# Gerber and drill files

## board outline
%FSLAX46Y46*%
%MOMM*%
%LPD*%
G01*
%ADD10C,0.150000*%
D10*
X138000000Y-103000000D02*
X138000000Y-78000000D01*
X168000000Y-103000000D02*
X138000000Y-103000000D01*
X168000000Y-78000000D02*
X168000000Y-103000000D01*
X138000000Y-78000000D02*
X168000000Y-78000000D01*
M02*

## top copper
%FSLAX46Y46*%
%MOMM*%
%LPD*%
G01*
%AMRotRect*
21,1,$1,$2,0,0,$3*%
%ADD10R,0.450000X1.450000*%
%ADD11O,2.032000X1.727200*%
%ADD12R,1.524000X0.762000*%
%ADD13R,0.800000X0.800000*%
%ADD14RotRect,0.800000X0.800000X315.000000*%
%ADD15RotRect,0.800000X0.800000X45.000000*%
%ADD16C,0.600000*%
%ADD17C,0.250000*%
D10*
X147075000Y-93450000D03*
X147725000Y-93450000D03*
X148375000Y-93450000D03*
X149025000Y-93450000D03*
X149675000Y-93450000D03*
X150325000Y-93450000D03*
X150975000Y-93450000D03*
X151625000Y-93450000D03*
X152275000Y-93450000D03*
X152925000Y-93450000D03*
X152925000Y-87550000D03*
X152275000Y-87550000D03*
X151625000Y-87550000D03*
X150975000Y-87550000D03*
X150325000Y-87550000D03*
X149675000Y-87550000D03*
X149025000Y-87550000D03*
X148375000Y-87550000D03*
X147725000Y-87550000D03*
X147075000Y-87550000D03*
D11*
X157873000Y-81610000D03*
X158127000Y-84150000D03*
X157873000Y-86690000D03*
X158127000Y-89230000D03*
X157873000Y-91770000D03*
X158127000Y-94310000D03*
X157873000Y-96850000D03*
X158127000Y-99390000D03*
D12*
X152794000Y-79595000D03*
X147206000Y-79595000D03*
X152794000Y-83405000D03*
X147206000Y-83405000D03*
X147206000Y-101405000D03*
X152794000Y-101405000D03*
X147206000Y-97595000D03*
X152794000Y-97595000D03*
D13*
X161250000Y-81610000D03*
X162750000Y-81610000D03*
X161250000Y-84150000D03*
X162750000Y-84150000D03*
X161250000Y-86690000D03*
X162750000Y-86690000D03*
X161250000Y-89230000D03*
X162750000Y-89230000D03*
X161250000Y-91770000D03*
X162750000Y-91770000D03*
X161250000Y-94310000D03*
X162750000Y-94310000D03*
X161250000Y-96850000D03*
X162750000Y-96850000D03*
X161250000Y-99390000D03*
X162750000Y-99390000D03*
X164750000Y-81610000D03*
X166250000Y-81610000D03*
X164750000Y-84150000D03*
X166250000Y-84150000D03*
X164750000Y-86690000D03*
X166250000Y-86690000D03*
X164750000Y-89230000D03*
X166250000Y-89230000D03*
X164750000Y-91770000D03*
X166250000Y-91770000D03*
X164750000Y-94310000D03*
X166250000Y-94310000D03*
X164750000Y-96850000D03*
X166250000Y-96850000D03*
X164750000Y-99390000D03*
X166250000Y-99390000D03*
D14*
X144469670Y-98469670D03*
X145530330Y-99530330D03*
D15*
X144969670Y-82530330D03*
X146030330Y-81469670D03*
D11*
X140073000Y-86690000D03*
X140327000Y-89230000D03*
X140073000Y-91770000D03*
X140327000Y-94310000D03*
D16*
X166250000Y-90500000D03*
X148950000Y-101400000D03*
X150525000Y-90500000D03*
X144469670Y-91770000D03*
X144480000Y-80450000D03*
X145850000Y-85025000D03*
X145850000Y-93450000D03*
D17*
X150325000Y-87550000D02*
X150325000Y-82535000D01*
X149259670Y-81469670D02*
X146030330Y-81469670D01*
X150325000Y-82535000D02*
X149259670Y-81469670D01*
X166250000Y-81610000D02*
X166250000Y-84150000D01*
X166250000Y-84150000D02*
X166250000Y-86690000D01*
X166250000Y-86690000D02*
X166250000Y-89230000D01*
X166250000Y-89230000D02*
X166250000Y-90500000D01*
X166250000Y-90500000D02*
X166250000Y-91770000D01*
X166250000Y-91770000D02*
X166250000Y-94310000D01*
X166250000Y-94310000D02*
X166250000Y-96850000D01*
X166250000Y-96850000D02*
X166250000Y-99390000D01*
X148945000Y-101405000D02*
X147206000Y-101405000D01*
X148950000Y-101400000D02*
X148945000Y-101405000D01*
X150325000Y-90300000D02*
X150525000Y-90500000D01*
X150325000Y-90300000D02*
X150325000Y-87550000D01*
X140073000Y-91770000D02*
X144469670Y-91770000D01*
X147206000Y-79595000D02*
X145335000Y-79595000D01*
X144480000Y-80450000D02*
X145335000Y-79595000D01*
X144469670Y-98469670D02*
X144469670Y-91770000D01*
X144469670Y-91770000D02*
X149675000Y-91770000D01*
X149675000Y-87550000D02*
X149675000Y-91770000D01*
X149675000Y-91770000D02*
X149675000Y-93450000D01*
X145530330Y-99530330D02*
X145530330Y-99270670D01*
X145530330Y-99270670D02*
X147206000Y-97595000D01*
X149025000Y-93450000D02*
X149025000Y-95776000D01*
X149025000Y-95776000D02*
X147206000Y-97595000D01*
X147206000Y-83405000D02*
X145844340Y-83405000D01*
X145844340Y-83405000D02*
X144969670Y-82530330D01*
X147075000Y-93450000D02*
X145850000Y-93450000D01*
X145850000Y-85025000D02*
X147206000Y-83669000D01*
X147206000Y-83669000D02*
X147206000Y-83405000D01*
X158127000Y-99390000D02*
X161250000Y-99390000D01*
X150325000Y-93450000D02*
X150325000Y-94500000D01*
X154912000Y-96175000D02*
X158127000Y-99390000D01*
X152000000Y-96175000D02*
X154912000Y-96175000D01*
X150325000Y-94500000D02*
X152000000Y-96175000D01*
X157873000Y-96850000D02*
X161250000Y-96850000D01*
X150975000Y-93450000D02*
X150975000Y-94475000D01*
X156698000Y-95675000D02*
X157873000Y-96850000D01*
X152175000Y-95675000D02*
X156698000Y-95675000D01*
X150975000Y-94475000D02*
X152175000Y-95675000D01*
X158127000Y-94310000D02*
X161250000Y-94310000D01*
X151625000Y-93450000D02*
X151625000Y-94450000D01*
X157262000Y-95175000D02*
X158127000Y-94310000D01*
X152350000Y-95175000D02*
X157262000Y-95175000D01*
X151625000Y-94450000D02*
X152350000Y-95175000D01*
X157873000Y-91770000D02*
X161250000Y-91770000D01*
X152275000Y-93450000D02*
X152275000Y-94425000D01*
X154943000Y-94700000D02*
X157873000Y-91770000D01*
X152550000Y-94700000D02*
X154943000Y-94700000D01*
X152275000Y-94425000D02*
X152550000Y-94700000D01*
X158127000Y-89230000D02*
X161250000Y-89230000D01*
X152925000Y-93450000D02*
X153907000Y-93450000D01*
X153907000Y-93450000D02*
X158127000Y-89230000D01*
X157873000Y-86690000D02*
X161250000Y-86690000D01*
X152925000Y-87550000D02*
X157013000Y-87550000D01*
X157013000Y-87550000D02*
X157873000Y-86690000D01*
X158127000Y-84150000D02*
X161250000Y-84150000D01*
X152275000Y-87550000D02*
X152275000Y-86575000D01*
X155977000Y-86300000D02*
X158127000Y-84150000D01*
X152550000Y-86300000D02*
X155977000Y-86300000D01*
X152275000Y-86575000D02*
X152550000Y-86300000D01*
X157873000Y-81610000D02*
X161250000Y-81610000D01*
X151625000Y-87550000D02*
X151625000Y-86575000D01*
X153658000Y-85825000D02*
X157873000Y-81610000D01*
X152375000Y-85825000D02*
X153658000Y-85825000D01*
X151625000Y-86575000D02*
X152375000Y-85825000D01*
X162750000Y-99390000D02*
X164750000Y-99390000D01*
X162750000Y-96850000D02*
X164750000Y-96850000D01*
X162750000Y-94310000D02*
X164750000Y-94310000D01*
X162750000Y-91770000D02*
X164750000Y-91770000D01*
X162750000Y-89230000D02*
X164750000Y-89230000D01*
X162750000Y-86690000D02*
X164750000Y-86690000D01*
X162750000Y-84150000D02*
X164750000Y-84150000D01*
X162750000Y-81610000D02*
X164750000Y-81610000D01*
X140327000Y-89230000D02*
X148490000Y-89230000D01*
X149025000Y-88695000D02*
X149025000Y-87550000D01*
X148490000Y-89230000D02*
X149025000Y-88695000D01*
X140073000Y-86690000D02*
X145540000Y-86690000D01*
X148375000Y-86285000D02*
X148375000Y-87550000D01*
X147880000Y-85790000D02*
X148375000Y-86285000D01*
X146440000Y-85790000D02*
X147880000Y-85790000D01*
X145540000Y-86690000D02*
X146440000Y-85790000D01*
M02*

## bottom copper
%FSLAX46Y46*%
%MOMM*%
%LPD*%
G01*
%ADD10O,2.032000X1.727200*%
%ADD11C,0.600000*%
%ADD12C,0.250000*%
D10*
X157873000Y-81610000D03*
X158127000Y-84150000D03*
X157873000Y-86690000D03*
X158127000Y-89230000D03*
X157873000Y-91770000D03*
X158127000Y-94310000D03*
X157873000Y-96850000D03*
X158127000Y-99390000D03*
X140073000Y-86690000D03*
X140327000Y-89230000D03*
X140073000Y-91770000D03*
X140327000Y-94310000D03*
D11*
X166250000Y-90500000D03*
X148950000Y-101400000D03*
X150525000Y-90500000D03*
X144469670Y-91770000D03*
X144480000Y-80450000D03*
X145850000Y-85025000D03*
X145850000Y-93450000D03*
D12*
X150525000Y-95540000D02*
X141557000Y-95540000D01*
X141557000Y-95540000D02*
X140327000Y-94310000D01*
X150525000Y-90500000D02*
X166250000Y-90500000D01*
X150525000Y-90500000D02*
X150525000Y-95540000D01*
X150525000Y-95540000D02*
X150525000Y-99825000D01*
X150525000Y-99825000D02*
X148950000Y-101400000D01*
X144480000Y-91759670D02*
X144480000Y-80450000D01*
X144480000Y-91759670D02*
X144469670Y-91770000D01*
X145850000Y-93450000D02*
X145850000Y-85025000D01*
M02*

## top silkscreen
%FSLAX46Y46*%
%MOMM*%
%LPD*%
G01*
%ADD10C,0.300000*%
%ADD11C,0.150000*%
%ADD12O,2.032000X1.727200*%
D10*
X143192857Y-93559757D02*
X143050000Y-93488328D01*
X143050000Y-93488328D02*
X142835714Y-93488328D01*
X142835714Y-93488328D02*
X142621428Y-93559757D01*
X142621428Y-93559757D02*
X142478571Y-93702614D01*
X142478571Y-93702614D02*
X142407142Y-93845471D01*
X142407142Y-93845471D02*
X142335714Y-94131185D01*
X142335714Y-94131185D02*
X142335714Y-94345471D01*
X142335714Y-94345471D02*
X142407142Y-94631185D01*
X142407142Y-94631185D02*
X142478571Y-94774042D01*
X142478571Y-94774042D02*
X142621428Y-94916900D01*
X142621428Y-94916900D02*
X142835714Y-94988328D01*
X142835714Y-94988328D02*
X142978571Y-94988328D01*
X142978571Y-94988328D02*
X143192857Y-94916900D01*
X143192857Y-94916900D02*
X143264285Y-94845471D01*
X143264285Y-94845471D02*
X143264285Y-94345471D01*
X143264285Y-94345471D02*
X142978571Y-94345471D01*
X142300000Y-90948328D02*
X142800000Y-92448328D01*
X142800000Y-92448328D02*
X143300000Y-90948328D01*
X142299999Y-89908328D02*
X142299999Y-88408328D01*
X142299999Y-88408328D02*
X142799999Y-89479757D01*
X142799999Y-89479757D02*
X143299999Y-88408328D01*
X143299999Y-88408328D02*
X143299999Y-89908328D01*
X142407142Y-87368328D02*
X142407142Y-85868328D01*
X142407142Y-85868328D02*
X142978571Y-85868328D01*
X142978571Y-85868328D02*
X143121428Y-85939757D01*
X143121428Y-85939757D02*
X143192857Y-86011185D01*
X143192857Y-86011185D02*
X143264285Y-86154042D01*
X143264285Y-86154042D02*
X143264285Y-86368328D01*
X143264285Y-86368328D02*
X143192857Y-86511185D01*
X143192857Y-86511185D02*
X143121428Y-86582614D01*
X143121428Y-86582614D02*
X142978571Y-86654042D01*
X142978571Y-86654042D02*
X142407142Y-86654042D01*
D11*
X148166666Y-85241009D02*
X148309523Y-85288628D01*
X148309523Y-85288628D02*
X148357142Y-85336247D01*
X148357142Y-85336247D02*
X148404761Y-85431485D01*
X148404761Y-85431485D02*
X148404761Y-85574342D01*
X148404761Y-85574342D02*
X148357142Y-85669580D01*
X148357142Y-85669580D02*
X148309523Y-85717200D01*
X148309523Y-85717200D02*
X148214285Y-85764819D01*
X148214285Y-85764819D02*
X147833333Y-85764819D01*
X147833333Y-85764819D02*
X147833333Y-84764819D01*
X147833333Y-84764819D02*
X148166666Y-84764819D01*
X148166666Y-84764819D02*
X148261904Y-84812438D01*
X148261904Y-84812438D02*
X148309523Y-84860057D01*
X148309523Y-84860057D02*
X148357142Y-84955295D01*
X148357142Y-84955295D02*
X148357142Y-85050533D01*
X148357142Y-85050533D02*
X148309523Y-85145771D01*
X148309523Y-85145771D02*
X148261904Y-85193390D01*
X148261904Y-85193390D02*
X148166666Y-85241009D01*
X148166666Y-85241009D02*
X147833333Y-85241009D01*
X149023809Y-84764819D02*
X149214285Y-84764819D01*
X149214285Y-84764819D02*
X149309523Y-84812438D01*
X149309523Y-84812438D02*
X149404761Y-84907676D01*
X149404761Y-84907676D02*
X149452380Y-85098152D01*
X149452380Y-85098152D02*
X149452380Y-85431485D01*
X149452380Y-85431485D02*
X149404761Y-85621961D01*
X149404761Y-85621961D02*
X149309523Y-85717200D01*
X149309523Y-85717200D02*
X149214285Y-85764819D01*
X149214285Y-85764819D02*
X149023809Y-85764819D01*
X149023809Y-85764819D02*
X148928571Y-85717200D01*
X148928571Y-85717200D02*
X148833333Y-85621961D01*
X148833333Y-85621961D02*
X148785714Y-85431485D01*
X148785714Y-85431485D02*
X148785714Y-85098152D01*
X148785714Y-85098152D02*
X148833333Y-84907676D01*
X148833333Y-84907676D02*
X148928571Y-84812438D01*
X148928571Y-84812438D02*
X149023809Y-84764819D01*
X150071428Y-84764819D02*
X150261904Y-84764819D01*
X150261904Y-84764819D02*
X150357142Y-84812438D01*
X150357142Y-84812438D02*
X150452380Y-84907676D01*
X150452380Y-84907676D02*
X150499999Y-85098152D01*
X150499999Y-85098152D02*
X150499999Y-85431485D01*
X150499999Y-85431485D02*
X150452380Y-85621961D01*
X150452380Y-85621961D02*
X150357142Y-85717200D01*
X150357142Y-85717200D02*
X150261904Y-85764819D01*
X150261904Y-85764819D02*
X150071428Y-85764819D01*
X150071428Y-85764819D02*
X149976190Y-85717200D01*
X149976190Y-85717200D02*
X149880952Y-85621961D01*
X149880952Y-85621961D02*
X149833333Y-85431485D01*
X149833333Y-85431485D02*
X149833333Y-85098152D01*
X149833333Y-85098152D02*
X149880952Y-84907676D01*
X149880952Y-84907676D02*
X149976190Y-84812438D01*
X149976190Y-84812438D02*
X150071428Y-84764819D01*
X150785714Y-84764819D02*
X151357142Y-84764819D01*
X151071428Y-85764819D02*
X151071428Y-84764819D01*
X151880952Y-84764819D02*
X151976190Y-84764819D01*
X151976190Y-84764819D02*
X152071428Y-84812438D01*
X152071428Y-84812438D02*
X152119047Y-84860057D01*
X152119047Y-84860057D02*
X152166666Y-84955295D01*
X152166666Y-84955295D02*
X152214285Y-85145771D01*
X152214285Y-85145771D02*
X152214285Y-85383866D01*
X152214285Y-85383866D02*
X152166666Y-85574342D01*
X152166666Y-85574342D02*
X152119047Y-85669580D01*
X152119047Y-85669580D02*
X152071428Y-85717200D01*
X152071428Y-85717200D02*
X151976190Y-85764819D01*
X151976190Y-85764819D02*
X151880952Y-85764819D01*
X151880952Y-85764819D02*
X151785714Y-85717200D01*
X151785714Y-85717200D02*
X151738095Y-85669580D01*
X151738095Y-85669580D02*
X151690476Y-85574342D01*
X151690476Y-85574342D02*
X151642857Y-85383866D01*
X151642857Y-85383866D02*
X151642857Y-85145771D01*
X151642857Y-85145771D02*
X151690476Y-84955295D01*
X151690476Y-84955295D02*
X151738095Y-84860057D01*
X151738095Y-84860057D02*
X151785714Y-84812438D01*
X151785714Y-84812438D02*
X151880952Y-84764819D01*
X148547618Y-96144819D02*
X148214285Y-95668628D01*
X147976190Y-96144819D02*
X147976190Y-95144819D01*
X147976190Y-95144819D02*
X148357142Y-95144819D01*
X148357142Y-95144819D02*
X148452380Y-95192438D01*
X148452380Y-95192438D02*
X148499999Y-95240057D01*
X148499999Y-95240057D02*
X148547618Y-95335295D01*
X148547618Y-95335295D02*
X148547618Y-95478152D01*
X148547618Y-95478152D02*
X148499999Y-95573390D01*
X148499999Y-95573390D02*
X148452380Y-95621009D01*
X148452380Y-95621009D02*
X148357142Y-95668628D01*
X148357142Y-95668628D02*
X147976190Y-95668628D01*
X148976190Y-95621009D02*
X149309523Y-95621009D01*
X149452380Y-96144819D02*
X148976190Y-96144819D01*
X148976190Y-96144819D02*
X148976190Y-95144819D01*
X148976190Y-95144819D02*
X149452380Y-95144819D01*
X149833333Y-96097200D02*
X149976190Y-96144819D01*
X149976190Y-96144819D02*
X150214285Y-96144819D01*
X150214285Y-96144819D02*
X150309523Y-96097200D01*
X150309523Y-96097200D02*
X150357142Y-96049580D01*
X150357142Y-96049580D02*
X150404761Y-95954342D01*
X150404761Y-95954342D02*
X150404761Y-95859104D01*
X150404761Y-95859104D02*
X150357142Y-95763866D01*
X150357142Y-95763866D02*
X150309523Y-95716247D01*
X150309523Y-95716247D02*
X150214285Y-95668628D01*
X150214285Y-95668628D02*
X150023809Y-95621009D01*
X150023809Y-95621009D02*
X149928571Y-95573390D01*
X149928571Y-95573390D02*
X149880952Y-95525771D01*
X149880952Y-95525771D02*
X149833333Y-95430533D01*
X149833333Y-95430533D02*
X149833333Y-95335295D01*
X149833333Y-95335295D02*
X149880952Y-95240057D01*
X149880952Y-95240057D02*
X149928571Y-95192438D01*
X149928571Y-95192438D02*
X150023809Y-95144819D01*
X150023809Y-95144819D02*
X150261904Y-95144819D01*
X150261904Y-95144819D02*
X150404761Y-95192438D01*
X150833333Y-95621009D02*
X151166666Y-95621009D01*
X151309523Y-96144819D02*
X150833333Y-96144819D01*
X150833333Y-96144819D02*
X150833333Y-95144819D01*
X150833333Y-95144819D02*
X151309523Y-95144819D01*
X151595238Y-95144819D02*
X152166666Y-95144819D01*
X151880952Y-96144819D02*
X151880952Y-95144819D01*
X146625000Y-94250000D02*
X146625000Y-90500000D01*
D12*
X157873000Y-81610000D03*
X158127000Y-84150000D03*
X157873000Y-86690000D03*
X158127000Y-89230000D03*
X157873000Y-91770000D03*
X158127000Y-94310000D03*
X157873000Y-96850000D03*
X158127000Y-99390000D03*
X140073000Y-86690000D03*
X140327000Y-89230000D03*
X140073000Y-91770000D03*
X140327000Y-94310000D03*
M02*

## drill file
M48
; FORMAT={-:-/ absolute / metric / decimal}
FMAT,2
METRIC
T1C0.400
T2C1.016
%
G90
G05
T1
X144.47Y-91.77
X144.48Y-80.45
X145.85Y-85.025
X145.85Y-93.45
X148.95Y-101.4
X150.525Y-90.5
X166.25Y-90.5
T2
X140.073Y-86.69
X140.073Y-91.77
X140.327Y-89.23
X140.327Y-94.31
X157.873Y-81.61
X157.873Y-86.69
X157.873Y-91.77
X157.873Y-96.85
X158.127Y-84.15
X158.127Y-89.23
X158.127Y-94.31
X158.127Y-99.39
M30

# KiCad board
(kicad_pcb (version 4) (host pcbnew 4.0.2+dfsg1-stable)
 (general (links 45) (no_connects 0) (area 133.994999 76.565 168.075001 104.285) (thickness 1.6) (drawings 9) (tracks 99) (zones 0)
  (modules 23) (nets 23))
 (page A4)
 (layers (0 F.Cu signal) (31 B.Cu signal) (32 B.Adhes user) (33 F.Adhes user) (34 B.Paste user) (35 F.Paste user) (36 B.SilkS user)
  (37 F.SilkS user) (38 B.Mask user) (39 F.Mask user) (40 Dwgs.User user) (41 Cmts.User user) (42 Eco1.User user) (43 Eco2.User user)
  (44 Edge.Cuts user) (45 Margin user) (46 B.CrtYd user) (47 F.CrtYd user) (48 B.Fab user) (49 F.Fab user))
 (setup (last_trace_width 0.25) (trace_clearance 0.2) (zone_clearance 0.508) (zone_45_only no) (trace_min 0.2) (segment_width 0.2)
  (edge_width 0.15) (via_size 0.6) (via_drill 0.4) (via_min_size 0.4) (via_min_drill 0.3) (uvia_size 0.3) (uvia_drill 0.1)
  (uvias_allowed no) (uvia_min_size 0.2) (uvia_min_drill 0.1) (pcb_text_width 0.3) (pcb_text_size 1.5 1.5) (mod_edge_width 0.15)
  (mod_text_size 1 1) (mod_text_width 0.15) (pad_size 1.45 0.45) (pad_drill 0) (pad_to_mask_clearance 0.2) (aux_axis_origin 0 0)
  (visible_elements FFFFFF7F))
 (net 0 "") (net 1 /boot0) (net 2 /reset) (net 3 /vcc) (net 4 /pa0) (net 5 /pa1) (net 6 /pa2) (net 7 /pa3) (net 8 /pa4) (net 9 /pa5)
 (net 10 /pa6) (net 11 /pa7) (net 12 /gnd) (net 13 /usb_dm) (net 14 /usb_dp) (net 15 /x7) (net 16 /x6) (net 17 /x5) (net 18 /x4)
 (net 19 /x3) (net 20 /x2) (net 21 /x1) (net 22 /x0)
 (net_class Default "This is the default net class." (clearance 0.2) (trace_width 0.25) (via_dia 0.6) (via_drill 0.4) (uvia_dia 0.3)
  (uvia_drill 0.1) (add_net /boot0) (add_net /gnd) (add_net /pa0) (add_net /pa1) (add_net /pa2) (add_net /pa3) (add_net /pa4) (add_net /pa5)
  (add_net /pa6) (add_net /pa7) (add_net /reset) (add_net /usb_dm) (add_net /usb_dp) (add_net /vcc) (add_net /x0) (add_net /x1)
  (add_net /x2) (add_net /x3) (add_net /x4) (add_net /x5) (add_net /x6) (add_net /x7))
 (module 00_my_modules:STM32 (layer F.Cu) (at 150 90.5 90)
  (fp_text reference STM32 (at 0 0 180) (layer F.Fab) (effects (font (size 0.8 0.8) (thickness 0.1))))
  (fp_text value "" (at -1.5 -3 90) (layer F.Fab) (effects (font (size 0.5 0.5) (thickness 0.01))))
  (fp_line (start -3.75 -3.375) (end 0 -3.375) (layer F.SilkS) (width 0.15))
  (pad BOOT smd rect (at -2.95 -2.925 90) (size 1.45 0.45) (layers F.Cu F.Paste F.Mask) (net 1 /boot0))
  (pad 2 smd rect (at -2.95 -2.275 90) (size 1.45 0.45) (layers F.Cu F.Paste F.Mask))
  (pad 3 smd rect (at -2.95 -1.625 90) (size 1.45 0.45) (layers F.Cu F.Paste F.Mask))
  (pad NRST smd rect (at -2.95 -0.975 90) (size 1.45 0.45) (layers F.Cu F.Paste F.Mask) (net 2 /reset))
  (pad VCC smd rect (at -2.95 -0.325 90) (size 1.45 0.45) (layers F.Cu F.Paste F.Mask) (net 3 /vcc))
  (pad PA0 smd rect (at -2.95 0.325 90) (size 1.45 0.45) (layers F.Cu F.Paste F.Mask) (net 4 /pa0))
  (pad PA1 smd rect (at -2.95 0.975 90) (size 1.45 0.45) (layers F.Cu F.Paste F.Mask) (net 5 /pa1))
  (pad PA2 smd rect (at -2.95 1.625 90) (size 1.45 0.45) (layers F.Cu F.Paste F.Mask) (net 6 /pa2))
  (pad PA3 smd rect (at -2.95 2.275 90) (size 1.45 0.45) (layers F.Cu F.Paste F.Mask) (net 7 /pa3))
  (pad PA4 smd rect (at -2.95 2.925 90) (size 1.45 0.45) (layers F.Cu F.Paste F.Mask) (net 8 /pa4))
  (pad PA5 smd rect (at 2.95 2.925 90) (size 1.45 0.45) (layers F.Cu F.Paste F.Mask) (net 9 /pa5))
  (pad PA6 smd rect (at 2.95 2.275 90) (size 1.45 0.45) (layers F.Cu F.Paste F.Mask) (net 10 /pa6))
  (pad PA7 smd rect (at 2.95 1.625 90) (size 1.45 0.45) (layers F.Cu F.Paste F.Mask) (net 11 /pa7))
  (pad PB1 smd rect (at 2.95 0.975 90) (size 1.45 0.45) (layers F.Cu F.Paste F.Mask))
  (pad GND smd rect (at 2.95 0.325 90) (size 1.45 0.45) (layers F.Cu F.Paste F.Mask) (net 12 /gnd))
  (pad VCC smd rect (at 2.95 -0.325 90) (size 1.45 0.45) (layers F.Cu F.Paste F.Mask) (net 3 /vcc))
  (pad DM smd rect (at 2.95 -0.975 90) (size 1.45 0.45) (layers F.Cu F.Paste F.Mask) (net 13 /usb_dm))
  (pad DP smd rect (at 2.95 -1.625 90) (size 1.45 0.45) (layers F.Cu F.Paste F.Mask) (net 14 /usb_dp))
  (pad DIO smd rect (at 2.95 -2.275 90) (size 1.45 0.45) (layers F.Cu F.Paste F.Mask))
  (pad CLK smd rect (at 2.95 -2.925 90) (size 1.45 0.45) (layers F.Cu F.Paste F.Mask)))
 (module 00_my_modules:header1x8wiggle (layer F.Cu) (at 158 90.5)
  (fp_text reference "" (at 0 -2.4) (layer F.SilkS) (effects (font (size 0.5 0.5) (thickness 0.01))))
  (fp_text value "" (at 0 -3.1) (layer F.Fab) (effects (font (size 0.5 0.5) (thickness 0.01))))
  (pad 7 thru_hole oval (at -0.127 -8.89) (size 2.032 1.7272) (drill 1.016) (layers *.Cu *.Mask F.SilkS) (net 11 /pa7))
  (pad 6 thru_hole oval (at 0.127 -6.35) (size 2.032 1.7272) (drill 1.016) (layers *.Cu *.Mask F.SilkS) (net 10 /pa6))
  (pad 5 thru_hole oval (at -0.127 -3.81) (size 2.032 1.7272) (drill 1.016) (layers *.Cu *.Mask F.SilkS) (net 9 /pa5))
  (pad 4 thru_hole oval (at 0.127 -1.27) (size 2.032 1.7272) (drill 1.016) (layers *.Cu *.Mask F.SilkS) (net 8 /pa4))
  (pad 3 thru_hole oval (at -0.127 1.27) (size 2.032 1.7272) (drill 1.016) (layers *.Cu *.Mask F.SilkS) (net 7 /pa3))
  (pad 2 thru_hole oval (at 0.127 3.81) (size 2.032 1.7272) (drill 1.016) (layers *.Cu *.Mask F.SilkS) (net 6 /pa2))
  (pad 1 thru_hole oval (at -0.127 6.35) (size 2.032 1.7272) (drill 1.016) (layers *.Cu *.Mask F.SilkS) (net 5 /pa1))
  (pad 0 thru_hole oval (at 0.127 8.89) (size 2.032 1.7272) (drill 1.016) (layers *.Cu *.Mask F.SilkS) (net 4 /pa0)))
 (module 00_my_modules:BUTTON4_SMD (layer F.Cu) (at 150 81.5 180)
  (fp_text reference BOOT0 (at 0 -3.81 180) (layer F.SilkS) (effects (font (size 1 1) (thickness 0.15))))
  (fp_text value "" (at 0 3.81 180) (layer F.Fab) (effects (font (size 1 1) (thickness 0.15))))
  (pad 1 smd rect (at -2.794 1.905 180) (size 1.524 0.762) (layers F.Cu F.Paste F.Mask))
  (pad 2 smd rect (at 2.794 1.905 180) (size 1.524 0.762) (layers F.Cu F.Paste F.Mask) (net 3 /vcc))
  (pad 3 smd rect (at -2.794 -1.905 180) (size 1.524 0.762) (layers F.Cu F.Paste F.Mask))
  (pad 4 smd rect (at 2.794 -1.905 180) (size 1.524 0.762) (layers F.Cu F.Paste F.Mask) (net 1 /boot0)))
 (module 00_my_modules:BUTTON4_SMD (layer F.Cu) (at 150 99.5)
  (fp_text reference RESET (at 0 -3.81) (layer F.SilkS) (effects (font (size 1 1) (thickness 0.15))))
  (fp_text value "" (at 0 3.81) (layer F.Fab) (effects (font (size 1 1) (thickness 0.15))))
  (pad 1 smd rect (at -2.794 1.905) (size 1.524 0.762) (layers F.Cu F.Paste F.Mask) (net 12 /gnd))
  (pad 2 smd rect (at 2.794 1.905) (size 1.524 0.762) (layers F.Cu F.Paste F.Mask))
  (pad 3 smd rect (at -2.794 -1.905) (size 1.524 0.762) (layers F.Cu F.Paste F.Mask) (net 2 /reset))
  (pad 4 smd rect (at 2.794 -1.905) (size 1.524 0.762) (layers F.Cu F.Paste F.Mask)))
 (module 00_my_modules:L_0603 (layer F.Cu) (at 162 81.61)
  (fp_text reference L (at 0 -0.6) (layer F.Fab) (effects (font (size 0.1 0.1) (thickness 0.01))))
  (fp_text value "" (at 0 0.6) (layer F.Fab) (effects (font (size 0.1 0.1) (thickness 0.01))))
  (pad 1 smd rect (at -0.75 0) (size 0.8 0.8) (layers F.Cu F.Paste F.Mask) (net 11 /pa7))
  (pad 2 smd rect (at 0.75 0) (size 0.8 0.8) (layers F.Cu F.Paste F.Mask) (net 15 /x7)))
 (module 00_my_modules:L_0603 (layer F.Cu) (at 162 84.15)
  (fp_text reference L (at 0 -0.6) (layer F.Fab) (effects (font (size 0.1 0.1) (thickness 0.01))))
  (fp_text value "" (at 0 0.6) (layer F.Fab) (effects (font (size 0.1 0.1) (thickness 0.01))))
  (pad 1 smd rect (at -0.75 0) (size 0.8 0.8) (layers F.Cu F.Paste F.Mask) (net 10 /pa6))
  (pad 2 smd rect (at 0.75 0) (size 0.8 0.8) (layers F.Cu F.Paste F.Mask) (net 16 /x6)))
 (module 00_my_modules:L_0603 (layer F.Cu) (at 162 86.69)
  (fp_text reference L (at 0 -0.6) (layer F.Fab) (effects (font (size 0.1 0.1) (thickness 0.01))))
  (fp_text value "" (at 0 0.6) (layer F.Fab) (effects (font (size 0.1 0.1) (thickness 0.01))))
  (pad 1 smd rect (at -0.75 0) (size 0.8 0.8) (layers F.Cu F.Paste F.Mask) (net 9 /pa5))
  (pad 2 smd rect (at 0.75 0) (size 0.8 0.8) (layers F.Cu F.Paste F.Mask) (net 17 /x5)))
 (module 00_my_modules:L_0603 (layer F.Cu) (at 162 89.23)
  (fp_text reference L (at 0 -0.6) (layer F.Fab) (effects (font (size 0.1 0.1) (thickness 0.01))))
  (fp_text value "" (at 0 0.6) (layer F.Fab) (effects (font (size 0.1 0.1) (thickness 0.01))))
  (pad 1 smd rect (at -0.75 0) (size 0.8 0.8) (layers F.Cu F.Paste F.Mask) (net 8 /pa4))
  (pad 4 smd rect (at 0.75 0) (size 0.8 0.8) (layers F.Cu F.Paste F.Mask) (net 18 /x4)))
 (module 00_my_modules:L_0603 (layer F.Cu) (at 162 91.77)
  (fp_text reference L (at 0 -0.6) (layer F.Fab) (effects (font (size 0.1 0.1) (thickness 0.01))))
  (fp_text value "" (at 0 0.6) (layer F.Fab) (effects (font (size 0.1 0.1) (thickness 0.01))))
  (pad 1 smd rect (at -0.75 0) (size 0.8 0.8) (layers F.Cu F.Paste F.Mask) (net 7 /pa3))
  (pad 2 smd rect (at 0.75 0) (size 0.8 0.8) (layers F.Cu F.Paste F.Mask) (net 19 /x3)))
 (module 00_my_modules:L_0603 (layer F.Cu) (at 162 94.31)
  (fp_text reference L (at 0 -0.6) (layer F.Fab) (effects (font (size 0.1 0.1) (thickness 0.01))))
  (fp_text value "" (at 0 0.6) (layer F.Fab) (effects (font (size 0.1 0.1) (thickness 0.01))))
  (pad 1 smd rect (at -0.75 0) (size 0.8 0.8) (layers F.Cu F.Paste F.Mask) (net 6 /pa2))
  (pad 2 smd rect (at 0.75 0) (size 0.8 0.8) (layers F.Cu F.Paste F.Mask) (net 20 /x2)))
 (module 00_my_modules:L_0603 (layer F.Cu) (at 162 96.85)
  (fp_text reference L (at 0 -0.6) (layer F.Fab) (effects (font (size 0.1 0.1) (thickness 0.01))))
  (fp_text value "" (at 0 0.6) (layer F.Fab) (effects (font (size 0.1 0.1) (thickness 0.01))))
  (pad 1 smd rect (at -0.75 0) (size 0.8 0.8) (layers F.Cu F.Paste F.Mask) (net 5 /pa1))
  (pad 2 smd rect (at 0.75 0) (size 0.8 0.8) (layers F.Cu F.Paste F.Mask) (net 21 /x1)))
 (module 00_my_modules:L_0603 (layer F.Cu) (at 162 99.39)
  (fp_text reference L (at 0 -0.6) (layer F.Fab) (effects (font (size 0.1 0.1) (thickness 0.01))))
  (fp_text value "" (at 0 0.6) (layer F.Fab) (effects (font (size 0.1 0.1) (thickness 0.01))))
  (pad 1 smd rect (at -0.75 0) (size 0.8 0.8) (layers F.Cu F.Paste F.Mask) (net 4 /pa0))
  (pad 2 smd rect (at 0.75 0) (size 0.8 0.8) (layers F.Cu F.Paste F.Mask) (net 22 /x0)))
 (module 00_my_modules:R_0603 (layer F.Cu) (at 165.5 81.61)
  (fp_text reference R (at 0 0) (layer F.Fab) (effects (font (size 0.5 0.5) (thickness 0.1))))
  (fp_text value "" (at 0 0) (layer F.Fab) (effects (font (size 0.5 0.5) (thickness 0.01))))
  (pad 1 smd rect (at -0.75 0) (size 0.8 0.8) (layers F.Cu F.Paste F.Mask) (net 15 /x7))
  (pad 2 smd rect (at 0.75 0) (size 0.8 0.8) (layers F.Cu F.Paste F.Mask) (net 12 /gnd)))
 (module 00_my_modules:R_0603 (layer F.Cu) (at 165.5 84.15)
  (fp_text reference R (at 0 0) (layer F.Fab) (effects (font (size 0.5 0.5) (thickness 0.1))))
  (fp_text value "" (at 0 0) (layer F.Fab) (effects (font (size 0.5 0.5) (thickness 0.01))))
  (pad 1 smd rect (at -0.75 0) (size 0.8 0.8) (layers F.Cu F.Paste F.Mask) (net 16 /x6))
  (pad 2 smd rect (at 0.75 0) (size 0.8 0.8) (layers F.Cu F.Paste F.Mask) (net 12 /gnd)))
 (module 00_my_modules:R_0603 (layer F.Cu) (at 165.5 86.69)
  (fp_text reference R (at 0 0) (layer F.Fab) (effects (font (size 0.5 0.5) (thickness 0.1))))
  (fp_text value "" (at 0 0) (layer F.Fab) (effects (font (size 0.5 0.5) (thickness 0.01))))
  (pad 1 smd rect (at -0.75 0) (size 0.8 0.8) (layers F.Cu F.Paste F.Mask) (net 17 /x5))
  (pad 2 smd rect (at 0.75 0) (size 0.8 0.8) (layers F.Cu F.Paste F.Mask) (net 12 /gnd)))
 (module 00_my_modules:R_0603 (layer F.Cu) (at 165.5 89.23)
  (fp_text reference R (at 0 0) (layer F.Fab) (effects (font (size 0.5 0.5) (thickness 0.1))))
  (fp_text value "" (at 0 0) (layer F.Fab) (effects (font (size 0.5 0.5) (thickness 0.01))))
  (pad 1 smd rect (at -0.75 0) (size 0.8 0.8) (layers F.Cu F.Paste F.Mask) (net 18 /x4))
  (pad 2 smd rect (at 0.75 0) (size 0.8 0.8) (layers F.Cu F.Paste F.Mask) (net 12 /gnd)))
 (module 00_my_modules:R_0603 (layer F.Cu) (at 165.5 91.77)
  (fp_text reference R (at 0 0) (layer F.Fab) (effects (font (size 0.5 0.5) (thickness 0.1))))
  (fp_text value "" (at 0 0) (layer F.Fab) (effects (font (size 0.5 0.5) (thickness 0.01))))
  (pad 1 smd rect (at -0.75 0) (size 0.8 0.8) (layers F.Cu F.Paste F.Mask) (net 19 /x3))
  (pad 2 smd rect (at 0.75 0) (size 0.8 0.8) (layers F.Cu F.Paste F.Mask) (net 12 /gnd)))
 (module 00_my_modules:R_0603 (layer F.Cu) (at 165.5 94.31)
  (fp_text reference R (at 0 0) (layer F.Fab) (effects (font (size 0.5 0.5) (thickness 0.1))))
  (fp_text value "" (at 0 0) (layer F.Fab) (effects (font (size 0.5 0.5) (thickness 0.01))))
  (pad 1 smd rect (at -0.75 0) (size 0.8 0.8) (layers F.Cu F.Paste F.Mask) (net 20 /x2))
  (pad 2 smd rect (at 0.75 0) (size 0.8 0.8) (layers F.Cu F.Paste F.Mask) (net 12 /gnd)))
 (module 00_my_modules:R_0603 (layer F.Cu) (at 165.5 96.85)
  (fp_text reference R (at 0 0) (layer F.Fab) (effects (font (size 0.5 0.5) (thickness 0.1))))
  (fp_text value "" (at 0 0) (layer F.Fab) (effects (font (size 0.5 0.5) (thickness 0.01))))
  (pad 1 smd rect (at -0.75 0) (size 0.8 0.8) (layers F.Cu F.Paste F.Mask) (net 21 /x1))
  (pad 2 smd rect (at 0.75 0) (size 0.8 0.8) (layers F.Cu F.Paste F.Mask) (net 12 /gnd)))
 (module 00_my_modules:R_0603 (layer F.Cu) (at 165.5 99.39)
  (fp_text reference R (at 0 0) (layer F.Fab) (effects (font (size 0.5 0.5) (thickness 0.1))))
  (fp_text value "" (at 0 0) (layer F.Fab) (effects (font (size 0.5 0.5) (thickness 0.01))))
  (pad 1 smd rect (at -0.75 0) (size 0.8 0.8) (layers F.Cu F.Paste F.Mask) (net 22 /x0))
  (pad 2 smd rect (at 0.75 0) (size 0.8 0.8) (layers F.Cu F.Paste F.Mask) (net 12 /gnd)))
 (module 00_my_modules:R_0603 (layer F.Cu) (at 145 99 315)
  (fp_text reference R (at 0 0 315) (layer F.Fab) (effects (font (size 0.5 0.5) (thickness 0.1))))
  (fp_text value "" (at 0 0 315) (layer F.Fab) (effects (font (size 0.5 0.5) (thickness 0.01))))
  (pad 1 smd rect (at -0.75 0 315) (size 0.8 0.8) (layers F.Cu F.Paste F.Mask) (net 3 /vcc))
  (pad 2 smd rect (at 0.75 0 315) (size 0.8 0.8) (layers F.Cu F.Paste F.Mask) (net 2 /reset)))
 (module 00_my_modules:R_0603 (layer F.Cu) (at 145.5 82 45)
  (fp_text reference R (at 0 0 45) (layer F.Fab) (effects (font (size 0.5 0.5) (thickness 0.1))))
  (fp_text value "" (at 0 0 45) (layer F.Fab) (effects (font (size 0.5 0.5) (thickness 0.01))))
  (pad 1 smd rect (at -0.75 0 45) (size 0.8 0.8) (layers F.Cu F.Paste F.Mask) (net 1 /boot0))
  (pad 2 smd rect (at 0.75 0 45) (size 0.8 0.8) (layers F.Cu F.Paste F.Mask) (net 12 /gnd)))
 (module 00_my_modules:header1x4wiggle (layer F.Cu) (at 140.2 90.5)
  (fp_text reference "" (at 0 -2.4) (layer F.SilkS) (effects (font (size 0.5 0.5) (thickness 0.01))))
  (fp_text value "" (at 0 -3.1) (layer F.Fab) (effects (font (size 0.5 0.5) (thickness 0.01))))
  (pad 1 thru_hole oval (at -0.127 -3.81) (size 2.032 1.7272) (drill 1.016) (layers *.Cu *.Mask F.SilkS) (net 14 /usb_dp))
  (pad 2 thru_hole oval (at 0.127 -1.27) (size 2.032 1.7272) (drill 1.016) (layers *.Cu *.Mask F.SilkS) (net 13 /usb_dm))
  (pad 3 thru_hole oval (at -0.127 1.27) (size 2.032 1.7272) (drill 1.016) (layers *.Cu *.Mask F.SilkS) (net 3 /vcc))
  (pad 4 thru_hole oval (at 0.127 3.81) (size 2.032 1.7272) (drill 1.016) (layers *.Cu *.Mask F.SilkS) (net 12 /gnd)))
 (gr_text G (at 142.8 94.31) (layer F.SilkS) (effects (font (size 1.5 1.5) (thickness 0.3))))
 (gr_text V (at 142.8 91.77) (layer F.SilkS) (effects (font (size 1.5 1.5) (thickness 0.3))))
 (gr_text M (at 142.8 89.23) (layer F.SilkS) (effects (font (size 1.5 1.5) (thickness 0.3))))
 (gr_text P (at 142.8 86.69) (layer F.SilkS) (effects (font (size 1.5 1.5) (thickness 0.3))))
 (gr_line (start 138 103) (end 138 78) (angle 90) (layer Edge.Cuts) (width 0.15))
 (gr_line (start 168 103) (end 138 103) (angle 90) (layer Edge.Cuts) (width 0.15))
 (gr_line (start 168 78) (end 168 103) (angle 90) (layer Edge.Cuts) (width 0.15))
 (gr_line (start 138 78) (end 168 78) (angle 90) (layer Edge.Cuts) (width 0.15))
 (segment (start 150.525 95.54) (end 141.557 95.54) (width 0.25) (layer B.Cu) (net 12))
 (segment (start 141.557 95.54) (end 140.327 94.31) (width 0.25) (layer B.Cu) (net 12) (status 800000))
 (segment (start 150.325 87.55) (end 150.325 82.535) (width 0.25) (layer F.Cu) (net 12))
 (segment (start 149.25967 81.46967) (end 146.03033 81.46967) (width 0.25) (layer F.Cu) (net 12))
 (segment (start 150.325 82.535) (end 149.25967 81.46967) (width 0.25) (layer F.Cu) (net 12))
 (segment (start 150.525 90.5) (end 166.25 90.5) (width 0.25) (layer B.Cu) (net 12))
 (via (at 166.25 90.5) (size 0.6) (drill 0.4) (layers F.Cu B.Cu) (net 12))
 (segment (start 166.25 81.61) (end 166.25 84.15) (width 0.25) (layer F.Cu) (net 12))
 (segment (start 166.25 84.15) (end 166.25 86.69) (width 0.25) (layer F.Cu) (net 12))
 (segment (start 166.25 86.69) (end 166.25 89.23) (width 0.25) (layer F.Cu) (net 12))
 (segment (start 166.25 89.23) (end 166.25 90.5) (width 0.25) (layer F.Cu) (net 12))
 (segment (start 166.25 90.5) (end 166.25 91.77) (width 0.25) (layer F.Cu) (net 12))
 (segment (start 166.25 91.77) (end 166.25 94.31) (width 0.25) (layer F.Cu) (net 12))
 (segment (start 166.25 94.31) (end 166.25 96.85) (width 0.25) (layer F.Cu) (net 12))
 (segment (start 166.25 96.85) (end 166.25 99.39) (width 0.25) (layer F.Cu) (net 12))
 (segment (start 150.525 90.5) (end 150.525 95.54) (width 0.25) (layer B.Cu) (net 12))
 (segment (start 150.525 95.54) (end 150.525 99.825) (width 0.25) (layer B.Cu) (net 12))
 (segment (start 148.945 101.405) (end 147.206 101.405) (width 0.25) (layer F.Cu) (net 12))
 (segment (start 148.95 101.4) (end 148.945 101.405) (width 0.25) (layer F.Cu) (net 12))
 (via (at 148.95 101.4) (size 0.6) (drill 0.4) (layers F.Cu B.Cu) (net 12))
 (segment (start 150.525 99.825) (end 148.95 101.4) (width 0.25) (layer B.Cu) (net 12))
 (segment (start 150.325 90.3) (end 150.525 90.5) (width 0.25) (layer F.Cu) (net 12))
 (via (at 150.525 90.5) (size 0.6) (drill 0.4) (layers F.Cu B.Cu) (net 12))
 (segment (start 150.325 90.3) (end 150.325 87.55) (width 0.25) (layer F.Cu) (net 12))
 (segment (start 140.073 91.77) (end 144.46967 91.77) (width 0.25) (layer F.Cu) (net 3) (status 400000))
 (via (at 144.46967 91.77) (size 0.6) (drill 0.4) (layers F.Cu B.Cu) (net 3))
 (segment (start 147.206 79.595) (end 145.335 79.595) (width 0.25) (layer F.Cu) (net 3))
 (segment (start 144.48 80.45) (end 145.335 79.595) (width 0.25) (layer F.Cu) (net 3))
 (via (at 144.48 80.45) (size 0.6) (drill 0.4) (layers F.Cu B.Cu) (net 3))
 (segment (start 144.48 91.75967) (end 144.48 80.45) (width 0.25) (layer B.Cu) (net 3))
 (segment (start 144.48 91.75967) (end 144.46967 91.77) (width 0.25) (layer B.Cu) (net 3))
 (segment (start 144.46967 98.46967) (end 144.46967 91.77) (width 0.25) (layer F.Cu) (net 3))
 (segment (start 144.46967 91.77) (end 149.675 91.77) (width 0.25) (layer F.Cu) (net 3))
 (segment (start 149.675 87.55) (end 149.675 91.77) (width 0.25) (layer F.Cu) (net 3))
 (segment (start 149.675 91.77) (end 149.675 93.45) (width 0.25) (layer F.Cu) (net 3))
 (segment (start 145.53033 99.53033) (end 145.53033 99.27067) (width 0.25) (layer F.Cu) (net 2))
 (segment (start 145.53033 99.27067) (end 147.206 97.595) (width 0.25) (layer F.Cu) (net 2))
 (segment (start 149.025 93.45) (end 149.025 95.776) (width 0.25) (layer F.Cu) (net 2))
 (segment (start 149.025 95.776) (end 147.206 97.595) (width 0.25) (layer F.Cu) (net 2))
 (segment (start 147.206 83.405) (end 145.84434 83.405) (width 0.25) (layer F.Cu) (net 1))
 (segment (start 145.84434 83.405) (end 144.96967 82.53033) (width 0.25) (layer F.Cu) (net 1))
 (segment (start 147.075 93.45) (end 145.85 93.45) (width 0.25) (layer F.Cu) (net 1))
 (segment (start 145.85 85.025) (end 147.206 83.669) (width 0.25) (layer F.Cu) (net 1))
 (via (at 145.85 85.025) (size 0.6) (drill 0.4) (layers F.Cu B.Cu) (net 1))
 (segment (start 145.85 93.45) (end 145.85 85.025) (width 0.25) (layer B.Cu) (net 1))
 (via (at 145.85 93.45) (size 0.6) (drill 0.4) (layers F.Cu B.Cu) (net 1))
 (segment (start 147.206 83.669) (end 147.206 83.405) (width 0.25) (layer F.Cu) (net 1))
 (segment (start 158.127 99.39) (end 161.25 99.39) (width 0.25) (layer F.Cu) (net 4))
 (segment (start 150.325 93.45) (end 150.325 94.5) (width 0.25) (layer F.Cu) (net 4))
 (segment (start 154.912 96.175) (end 158.127 99.39) (width 0.25) (layer F.Cu) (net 4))
 (segment (start 152 96.175) (end 154.912 96.175) (width 0.25) (layer F.Cu) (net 4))
 (segment (start 150.325 94.5) (end 152 96.175) (width 0.25) (layer F.Cu) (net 4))
 (segment (start 157.873 96.85) (end 161.25 96.85) (width 0.25) (layer F.Cu) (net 5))
 (segment (start 150.975 93.45) (end 150.975 94.475) (width 0.25) (layer F.Cu) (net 5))
 (segment (start 156.698 95.675) (end 157.873 96.85) (width 0.25) (layer F.Cu) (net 5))
 (segment (start 152.175 95.675) (end 156.698 95.675) (width 0.25) (layer F.Cu) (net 5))
 (segment (start 150.975 94.475) (end 152.175 95.675) (width 0.25) (layer F.Cu) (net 5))
 (segment (start 158.127 94.31) (end 161.25 94.31) (width 0.25) (layer F.Cu) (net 6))
 (segment (start 151.625 93.45) (end 151.625 94.45) (width 0.25) (layer F.Cu) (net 6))
 (segment (start 157.262 95.175) (end 158.127 94.31) (width 0.25) (layer F.Cu) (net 6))
 (segment (start 152.35 95.175) (end 157.262 95.175) (width 0.25) (layer F.Cu) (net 6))
 (segment (start 151.625 94.45) (end 152.35 95.175) (width 0.25) (layer F.Cu) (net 6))
 (segment (start 157.873 91.77) (end 161.25 91.77) (width 0.25) (layer F.Cu) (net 7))
 (segment (start 152.275 93.45) (end 152.275 94.425) (width 0.25) (layer F.Cu) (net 7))
 (segment (start 154.943 94.7) (end 157.873 91.77) (width 0.25) (layer F.Cu) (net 7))
 (segment (start 152.55 94.7) (end 154.943 94.7) (width 0.25) (layer F.Cu) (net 7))
 (segment (start 152.275 94.425) (end 152.55 94.7) (width 0.25) (layer F.Cu) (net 7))
 (segment (start 158.127 89.23) (end 161.25 89.23) (width 0.25) (layer F.Cu) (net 8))
 (segment (start 152.925 93.45) (end 153.907 93.45) (width 0.25) (layer F.Cu) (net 8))
 (segment (start 153.907 93.45) (end 158.127 89.23) (width 0.25) (layer F.Cu) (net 8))
 (segment (start 157.873 86.69) (end 161.25 86.69) (width 0.25) (layer F.Cu) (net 9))
 (segment (start 152.925 87.55) (end 157.013 87.55) (width 0.25) (layer F.Cu) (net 9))
 (segment (start 157.013 87.55) (end 157.873 86.69) (width 0.25) (layer F.Cu) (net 9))
 (segment (start 158.127 84.15) (end 161.25 84.15) (width 0.25) (layer F.Cu) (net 10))
 (segment (start 152.275 87.55) (end 152.275 86.575) (width 0.25) (layer F.Cu) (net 10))
 (segment (start 155.977 86.3) (end 158.127 84.15) (width 0.25) (layer F.Cu) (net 10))
 (segment (start 152.55 86.3) (end 155.977 86.3) (width 0.25) (layer F.Cu) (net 10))
 (segment (start 152.275 86.575) (end 152.55 86.3) (width 0.25) (layer F.Cu) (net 10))
 (segment (start 157.873 81.61) (end 161.25 81.61) (width 0.25) (layer F.Cu) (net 11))
 (segment (start 151.625 87.55) (end 151.625 86.575) (width 0.25) (layer F.Cu) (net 11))
 (segment (start 153.658 85.825) (end 157.873 81.61) (width 0.25) (layer F.Cu) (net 11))
 (segment (start 152.375 85.825) (end 153.658 85.825) (width 0.25) (layer F.Cu) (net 11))
 (segment (start 151.625 86.575) (end 152.375 85.825) (width 0.25) (layer F.Cu) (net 11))
 (segment (start 162.75 99.39) (end 164.75 99.39) (width 0.25) (layer F.Cu) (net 22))
 (segment (start 162.75 96.85) (end 164.75 96.85) (width 0.25) (layer F.Cu) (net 21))
 (segment (start 162.75 94.31) (end 164.75 94.31) (width 0.25) (layer F.Cu) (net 20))
 (segment (start 162.75 91.77) (end 164.75 91.77) (width 0.25) (layer F.Cu) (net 19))
 (segment (start 162.75 89.23) (end 164.75 89.23) (width 0.25) (layer F.Cu) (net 18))
 (segment (start 162.75 86.69) (end 164.75 86.69) (width 0.25) (layer F.Cu) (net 17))
 (segment (start 162.75 84.15) (end 164.75 84.15) (width 0.25) (layer F.Cu) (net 16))
 (segment (start 162.75 81.61) (end 164.75 81.61) (width 0.25) (layer F.Cu) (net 15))
 (segment (start 140.327 89.23) (end 148.49 89.23) (width 0.25) (layer F.Cu) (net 13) (status 400000))
 (segment (start 149.025 88.695) (end 149.025 87.55) (width 0.25) (layer F.Cu) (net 13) (status 800000))
 (segment (start 148.49 89.23) (end 149.025 88.695) (width 0.25) (layer F.Cu) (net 13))
 (segment (start 140.073 86.69) (end 145.54 86.69) (width 0.25) (layer F.Cu) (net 14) (status 400000))
 (segment (start 148.375 86.285) (end 148.375 87.55) (width 0.25) (layer F.Cu) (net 14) (status 800000))
 (segment (start 147.88 85.79) (end 148.375 86.285) (width 0.25) (layer F.Cu) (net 14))
 (segment (start 146.44 85.79) (end 147.88 85.79) (width 0.25) (layer F.Cu) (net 14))
 (segment (start 145.54 86.69) (end 146.44 85.79) (width 0.25) (layer F.Cu) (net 14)))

